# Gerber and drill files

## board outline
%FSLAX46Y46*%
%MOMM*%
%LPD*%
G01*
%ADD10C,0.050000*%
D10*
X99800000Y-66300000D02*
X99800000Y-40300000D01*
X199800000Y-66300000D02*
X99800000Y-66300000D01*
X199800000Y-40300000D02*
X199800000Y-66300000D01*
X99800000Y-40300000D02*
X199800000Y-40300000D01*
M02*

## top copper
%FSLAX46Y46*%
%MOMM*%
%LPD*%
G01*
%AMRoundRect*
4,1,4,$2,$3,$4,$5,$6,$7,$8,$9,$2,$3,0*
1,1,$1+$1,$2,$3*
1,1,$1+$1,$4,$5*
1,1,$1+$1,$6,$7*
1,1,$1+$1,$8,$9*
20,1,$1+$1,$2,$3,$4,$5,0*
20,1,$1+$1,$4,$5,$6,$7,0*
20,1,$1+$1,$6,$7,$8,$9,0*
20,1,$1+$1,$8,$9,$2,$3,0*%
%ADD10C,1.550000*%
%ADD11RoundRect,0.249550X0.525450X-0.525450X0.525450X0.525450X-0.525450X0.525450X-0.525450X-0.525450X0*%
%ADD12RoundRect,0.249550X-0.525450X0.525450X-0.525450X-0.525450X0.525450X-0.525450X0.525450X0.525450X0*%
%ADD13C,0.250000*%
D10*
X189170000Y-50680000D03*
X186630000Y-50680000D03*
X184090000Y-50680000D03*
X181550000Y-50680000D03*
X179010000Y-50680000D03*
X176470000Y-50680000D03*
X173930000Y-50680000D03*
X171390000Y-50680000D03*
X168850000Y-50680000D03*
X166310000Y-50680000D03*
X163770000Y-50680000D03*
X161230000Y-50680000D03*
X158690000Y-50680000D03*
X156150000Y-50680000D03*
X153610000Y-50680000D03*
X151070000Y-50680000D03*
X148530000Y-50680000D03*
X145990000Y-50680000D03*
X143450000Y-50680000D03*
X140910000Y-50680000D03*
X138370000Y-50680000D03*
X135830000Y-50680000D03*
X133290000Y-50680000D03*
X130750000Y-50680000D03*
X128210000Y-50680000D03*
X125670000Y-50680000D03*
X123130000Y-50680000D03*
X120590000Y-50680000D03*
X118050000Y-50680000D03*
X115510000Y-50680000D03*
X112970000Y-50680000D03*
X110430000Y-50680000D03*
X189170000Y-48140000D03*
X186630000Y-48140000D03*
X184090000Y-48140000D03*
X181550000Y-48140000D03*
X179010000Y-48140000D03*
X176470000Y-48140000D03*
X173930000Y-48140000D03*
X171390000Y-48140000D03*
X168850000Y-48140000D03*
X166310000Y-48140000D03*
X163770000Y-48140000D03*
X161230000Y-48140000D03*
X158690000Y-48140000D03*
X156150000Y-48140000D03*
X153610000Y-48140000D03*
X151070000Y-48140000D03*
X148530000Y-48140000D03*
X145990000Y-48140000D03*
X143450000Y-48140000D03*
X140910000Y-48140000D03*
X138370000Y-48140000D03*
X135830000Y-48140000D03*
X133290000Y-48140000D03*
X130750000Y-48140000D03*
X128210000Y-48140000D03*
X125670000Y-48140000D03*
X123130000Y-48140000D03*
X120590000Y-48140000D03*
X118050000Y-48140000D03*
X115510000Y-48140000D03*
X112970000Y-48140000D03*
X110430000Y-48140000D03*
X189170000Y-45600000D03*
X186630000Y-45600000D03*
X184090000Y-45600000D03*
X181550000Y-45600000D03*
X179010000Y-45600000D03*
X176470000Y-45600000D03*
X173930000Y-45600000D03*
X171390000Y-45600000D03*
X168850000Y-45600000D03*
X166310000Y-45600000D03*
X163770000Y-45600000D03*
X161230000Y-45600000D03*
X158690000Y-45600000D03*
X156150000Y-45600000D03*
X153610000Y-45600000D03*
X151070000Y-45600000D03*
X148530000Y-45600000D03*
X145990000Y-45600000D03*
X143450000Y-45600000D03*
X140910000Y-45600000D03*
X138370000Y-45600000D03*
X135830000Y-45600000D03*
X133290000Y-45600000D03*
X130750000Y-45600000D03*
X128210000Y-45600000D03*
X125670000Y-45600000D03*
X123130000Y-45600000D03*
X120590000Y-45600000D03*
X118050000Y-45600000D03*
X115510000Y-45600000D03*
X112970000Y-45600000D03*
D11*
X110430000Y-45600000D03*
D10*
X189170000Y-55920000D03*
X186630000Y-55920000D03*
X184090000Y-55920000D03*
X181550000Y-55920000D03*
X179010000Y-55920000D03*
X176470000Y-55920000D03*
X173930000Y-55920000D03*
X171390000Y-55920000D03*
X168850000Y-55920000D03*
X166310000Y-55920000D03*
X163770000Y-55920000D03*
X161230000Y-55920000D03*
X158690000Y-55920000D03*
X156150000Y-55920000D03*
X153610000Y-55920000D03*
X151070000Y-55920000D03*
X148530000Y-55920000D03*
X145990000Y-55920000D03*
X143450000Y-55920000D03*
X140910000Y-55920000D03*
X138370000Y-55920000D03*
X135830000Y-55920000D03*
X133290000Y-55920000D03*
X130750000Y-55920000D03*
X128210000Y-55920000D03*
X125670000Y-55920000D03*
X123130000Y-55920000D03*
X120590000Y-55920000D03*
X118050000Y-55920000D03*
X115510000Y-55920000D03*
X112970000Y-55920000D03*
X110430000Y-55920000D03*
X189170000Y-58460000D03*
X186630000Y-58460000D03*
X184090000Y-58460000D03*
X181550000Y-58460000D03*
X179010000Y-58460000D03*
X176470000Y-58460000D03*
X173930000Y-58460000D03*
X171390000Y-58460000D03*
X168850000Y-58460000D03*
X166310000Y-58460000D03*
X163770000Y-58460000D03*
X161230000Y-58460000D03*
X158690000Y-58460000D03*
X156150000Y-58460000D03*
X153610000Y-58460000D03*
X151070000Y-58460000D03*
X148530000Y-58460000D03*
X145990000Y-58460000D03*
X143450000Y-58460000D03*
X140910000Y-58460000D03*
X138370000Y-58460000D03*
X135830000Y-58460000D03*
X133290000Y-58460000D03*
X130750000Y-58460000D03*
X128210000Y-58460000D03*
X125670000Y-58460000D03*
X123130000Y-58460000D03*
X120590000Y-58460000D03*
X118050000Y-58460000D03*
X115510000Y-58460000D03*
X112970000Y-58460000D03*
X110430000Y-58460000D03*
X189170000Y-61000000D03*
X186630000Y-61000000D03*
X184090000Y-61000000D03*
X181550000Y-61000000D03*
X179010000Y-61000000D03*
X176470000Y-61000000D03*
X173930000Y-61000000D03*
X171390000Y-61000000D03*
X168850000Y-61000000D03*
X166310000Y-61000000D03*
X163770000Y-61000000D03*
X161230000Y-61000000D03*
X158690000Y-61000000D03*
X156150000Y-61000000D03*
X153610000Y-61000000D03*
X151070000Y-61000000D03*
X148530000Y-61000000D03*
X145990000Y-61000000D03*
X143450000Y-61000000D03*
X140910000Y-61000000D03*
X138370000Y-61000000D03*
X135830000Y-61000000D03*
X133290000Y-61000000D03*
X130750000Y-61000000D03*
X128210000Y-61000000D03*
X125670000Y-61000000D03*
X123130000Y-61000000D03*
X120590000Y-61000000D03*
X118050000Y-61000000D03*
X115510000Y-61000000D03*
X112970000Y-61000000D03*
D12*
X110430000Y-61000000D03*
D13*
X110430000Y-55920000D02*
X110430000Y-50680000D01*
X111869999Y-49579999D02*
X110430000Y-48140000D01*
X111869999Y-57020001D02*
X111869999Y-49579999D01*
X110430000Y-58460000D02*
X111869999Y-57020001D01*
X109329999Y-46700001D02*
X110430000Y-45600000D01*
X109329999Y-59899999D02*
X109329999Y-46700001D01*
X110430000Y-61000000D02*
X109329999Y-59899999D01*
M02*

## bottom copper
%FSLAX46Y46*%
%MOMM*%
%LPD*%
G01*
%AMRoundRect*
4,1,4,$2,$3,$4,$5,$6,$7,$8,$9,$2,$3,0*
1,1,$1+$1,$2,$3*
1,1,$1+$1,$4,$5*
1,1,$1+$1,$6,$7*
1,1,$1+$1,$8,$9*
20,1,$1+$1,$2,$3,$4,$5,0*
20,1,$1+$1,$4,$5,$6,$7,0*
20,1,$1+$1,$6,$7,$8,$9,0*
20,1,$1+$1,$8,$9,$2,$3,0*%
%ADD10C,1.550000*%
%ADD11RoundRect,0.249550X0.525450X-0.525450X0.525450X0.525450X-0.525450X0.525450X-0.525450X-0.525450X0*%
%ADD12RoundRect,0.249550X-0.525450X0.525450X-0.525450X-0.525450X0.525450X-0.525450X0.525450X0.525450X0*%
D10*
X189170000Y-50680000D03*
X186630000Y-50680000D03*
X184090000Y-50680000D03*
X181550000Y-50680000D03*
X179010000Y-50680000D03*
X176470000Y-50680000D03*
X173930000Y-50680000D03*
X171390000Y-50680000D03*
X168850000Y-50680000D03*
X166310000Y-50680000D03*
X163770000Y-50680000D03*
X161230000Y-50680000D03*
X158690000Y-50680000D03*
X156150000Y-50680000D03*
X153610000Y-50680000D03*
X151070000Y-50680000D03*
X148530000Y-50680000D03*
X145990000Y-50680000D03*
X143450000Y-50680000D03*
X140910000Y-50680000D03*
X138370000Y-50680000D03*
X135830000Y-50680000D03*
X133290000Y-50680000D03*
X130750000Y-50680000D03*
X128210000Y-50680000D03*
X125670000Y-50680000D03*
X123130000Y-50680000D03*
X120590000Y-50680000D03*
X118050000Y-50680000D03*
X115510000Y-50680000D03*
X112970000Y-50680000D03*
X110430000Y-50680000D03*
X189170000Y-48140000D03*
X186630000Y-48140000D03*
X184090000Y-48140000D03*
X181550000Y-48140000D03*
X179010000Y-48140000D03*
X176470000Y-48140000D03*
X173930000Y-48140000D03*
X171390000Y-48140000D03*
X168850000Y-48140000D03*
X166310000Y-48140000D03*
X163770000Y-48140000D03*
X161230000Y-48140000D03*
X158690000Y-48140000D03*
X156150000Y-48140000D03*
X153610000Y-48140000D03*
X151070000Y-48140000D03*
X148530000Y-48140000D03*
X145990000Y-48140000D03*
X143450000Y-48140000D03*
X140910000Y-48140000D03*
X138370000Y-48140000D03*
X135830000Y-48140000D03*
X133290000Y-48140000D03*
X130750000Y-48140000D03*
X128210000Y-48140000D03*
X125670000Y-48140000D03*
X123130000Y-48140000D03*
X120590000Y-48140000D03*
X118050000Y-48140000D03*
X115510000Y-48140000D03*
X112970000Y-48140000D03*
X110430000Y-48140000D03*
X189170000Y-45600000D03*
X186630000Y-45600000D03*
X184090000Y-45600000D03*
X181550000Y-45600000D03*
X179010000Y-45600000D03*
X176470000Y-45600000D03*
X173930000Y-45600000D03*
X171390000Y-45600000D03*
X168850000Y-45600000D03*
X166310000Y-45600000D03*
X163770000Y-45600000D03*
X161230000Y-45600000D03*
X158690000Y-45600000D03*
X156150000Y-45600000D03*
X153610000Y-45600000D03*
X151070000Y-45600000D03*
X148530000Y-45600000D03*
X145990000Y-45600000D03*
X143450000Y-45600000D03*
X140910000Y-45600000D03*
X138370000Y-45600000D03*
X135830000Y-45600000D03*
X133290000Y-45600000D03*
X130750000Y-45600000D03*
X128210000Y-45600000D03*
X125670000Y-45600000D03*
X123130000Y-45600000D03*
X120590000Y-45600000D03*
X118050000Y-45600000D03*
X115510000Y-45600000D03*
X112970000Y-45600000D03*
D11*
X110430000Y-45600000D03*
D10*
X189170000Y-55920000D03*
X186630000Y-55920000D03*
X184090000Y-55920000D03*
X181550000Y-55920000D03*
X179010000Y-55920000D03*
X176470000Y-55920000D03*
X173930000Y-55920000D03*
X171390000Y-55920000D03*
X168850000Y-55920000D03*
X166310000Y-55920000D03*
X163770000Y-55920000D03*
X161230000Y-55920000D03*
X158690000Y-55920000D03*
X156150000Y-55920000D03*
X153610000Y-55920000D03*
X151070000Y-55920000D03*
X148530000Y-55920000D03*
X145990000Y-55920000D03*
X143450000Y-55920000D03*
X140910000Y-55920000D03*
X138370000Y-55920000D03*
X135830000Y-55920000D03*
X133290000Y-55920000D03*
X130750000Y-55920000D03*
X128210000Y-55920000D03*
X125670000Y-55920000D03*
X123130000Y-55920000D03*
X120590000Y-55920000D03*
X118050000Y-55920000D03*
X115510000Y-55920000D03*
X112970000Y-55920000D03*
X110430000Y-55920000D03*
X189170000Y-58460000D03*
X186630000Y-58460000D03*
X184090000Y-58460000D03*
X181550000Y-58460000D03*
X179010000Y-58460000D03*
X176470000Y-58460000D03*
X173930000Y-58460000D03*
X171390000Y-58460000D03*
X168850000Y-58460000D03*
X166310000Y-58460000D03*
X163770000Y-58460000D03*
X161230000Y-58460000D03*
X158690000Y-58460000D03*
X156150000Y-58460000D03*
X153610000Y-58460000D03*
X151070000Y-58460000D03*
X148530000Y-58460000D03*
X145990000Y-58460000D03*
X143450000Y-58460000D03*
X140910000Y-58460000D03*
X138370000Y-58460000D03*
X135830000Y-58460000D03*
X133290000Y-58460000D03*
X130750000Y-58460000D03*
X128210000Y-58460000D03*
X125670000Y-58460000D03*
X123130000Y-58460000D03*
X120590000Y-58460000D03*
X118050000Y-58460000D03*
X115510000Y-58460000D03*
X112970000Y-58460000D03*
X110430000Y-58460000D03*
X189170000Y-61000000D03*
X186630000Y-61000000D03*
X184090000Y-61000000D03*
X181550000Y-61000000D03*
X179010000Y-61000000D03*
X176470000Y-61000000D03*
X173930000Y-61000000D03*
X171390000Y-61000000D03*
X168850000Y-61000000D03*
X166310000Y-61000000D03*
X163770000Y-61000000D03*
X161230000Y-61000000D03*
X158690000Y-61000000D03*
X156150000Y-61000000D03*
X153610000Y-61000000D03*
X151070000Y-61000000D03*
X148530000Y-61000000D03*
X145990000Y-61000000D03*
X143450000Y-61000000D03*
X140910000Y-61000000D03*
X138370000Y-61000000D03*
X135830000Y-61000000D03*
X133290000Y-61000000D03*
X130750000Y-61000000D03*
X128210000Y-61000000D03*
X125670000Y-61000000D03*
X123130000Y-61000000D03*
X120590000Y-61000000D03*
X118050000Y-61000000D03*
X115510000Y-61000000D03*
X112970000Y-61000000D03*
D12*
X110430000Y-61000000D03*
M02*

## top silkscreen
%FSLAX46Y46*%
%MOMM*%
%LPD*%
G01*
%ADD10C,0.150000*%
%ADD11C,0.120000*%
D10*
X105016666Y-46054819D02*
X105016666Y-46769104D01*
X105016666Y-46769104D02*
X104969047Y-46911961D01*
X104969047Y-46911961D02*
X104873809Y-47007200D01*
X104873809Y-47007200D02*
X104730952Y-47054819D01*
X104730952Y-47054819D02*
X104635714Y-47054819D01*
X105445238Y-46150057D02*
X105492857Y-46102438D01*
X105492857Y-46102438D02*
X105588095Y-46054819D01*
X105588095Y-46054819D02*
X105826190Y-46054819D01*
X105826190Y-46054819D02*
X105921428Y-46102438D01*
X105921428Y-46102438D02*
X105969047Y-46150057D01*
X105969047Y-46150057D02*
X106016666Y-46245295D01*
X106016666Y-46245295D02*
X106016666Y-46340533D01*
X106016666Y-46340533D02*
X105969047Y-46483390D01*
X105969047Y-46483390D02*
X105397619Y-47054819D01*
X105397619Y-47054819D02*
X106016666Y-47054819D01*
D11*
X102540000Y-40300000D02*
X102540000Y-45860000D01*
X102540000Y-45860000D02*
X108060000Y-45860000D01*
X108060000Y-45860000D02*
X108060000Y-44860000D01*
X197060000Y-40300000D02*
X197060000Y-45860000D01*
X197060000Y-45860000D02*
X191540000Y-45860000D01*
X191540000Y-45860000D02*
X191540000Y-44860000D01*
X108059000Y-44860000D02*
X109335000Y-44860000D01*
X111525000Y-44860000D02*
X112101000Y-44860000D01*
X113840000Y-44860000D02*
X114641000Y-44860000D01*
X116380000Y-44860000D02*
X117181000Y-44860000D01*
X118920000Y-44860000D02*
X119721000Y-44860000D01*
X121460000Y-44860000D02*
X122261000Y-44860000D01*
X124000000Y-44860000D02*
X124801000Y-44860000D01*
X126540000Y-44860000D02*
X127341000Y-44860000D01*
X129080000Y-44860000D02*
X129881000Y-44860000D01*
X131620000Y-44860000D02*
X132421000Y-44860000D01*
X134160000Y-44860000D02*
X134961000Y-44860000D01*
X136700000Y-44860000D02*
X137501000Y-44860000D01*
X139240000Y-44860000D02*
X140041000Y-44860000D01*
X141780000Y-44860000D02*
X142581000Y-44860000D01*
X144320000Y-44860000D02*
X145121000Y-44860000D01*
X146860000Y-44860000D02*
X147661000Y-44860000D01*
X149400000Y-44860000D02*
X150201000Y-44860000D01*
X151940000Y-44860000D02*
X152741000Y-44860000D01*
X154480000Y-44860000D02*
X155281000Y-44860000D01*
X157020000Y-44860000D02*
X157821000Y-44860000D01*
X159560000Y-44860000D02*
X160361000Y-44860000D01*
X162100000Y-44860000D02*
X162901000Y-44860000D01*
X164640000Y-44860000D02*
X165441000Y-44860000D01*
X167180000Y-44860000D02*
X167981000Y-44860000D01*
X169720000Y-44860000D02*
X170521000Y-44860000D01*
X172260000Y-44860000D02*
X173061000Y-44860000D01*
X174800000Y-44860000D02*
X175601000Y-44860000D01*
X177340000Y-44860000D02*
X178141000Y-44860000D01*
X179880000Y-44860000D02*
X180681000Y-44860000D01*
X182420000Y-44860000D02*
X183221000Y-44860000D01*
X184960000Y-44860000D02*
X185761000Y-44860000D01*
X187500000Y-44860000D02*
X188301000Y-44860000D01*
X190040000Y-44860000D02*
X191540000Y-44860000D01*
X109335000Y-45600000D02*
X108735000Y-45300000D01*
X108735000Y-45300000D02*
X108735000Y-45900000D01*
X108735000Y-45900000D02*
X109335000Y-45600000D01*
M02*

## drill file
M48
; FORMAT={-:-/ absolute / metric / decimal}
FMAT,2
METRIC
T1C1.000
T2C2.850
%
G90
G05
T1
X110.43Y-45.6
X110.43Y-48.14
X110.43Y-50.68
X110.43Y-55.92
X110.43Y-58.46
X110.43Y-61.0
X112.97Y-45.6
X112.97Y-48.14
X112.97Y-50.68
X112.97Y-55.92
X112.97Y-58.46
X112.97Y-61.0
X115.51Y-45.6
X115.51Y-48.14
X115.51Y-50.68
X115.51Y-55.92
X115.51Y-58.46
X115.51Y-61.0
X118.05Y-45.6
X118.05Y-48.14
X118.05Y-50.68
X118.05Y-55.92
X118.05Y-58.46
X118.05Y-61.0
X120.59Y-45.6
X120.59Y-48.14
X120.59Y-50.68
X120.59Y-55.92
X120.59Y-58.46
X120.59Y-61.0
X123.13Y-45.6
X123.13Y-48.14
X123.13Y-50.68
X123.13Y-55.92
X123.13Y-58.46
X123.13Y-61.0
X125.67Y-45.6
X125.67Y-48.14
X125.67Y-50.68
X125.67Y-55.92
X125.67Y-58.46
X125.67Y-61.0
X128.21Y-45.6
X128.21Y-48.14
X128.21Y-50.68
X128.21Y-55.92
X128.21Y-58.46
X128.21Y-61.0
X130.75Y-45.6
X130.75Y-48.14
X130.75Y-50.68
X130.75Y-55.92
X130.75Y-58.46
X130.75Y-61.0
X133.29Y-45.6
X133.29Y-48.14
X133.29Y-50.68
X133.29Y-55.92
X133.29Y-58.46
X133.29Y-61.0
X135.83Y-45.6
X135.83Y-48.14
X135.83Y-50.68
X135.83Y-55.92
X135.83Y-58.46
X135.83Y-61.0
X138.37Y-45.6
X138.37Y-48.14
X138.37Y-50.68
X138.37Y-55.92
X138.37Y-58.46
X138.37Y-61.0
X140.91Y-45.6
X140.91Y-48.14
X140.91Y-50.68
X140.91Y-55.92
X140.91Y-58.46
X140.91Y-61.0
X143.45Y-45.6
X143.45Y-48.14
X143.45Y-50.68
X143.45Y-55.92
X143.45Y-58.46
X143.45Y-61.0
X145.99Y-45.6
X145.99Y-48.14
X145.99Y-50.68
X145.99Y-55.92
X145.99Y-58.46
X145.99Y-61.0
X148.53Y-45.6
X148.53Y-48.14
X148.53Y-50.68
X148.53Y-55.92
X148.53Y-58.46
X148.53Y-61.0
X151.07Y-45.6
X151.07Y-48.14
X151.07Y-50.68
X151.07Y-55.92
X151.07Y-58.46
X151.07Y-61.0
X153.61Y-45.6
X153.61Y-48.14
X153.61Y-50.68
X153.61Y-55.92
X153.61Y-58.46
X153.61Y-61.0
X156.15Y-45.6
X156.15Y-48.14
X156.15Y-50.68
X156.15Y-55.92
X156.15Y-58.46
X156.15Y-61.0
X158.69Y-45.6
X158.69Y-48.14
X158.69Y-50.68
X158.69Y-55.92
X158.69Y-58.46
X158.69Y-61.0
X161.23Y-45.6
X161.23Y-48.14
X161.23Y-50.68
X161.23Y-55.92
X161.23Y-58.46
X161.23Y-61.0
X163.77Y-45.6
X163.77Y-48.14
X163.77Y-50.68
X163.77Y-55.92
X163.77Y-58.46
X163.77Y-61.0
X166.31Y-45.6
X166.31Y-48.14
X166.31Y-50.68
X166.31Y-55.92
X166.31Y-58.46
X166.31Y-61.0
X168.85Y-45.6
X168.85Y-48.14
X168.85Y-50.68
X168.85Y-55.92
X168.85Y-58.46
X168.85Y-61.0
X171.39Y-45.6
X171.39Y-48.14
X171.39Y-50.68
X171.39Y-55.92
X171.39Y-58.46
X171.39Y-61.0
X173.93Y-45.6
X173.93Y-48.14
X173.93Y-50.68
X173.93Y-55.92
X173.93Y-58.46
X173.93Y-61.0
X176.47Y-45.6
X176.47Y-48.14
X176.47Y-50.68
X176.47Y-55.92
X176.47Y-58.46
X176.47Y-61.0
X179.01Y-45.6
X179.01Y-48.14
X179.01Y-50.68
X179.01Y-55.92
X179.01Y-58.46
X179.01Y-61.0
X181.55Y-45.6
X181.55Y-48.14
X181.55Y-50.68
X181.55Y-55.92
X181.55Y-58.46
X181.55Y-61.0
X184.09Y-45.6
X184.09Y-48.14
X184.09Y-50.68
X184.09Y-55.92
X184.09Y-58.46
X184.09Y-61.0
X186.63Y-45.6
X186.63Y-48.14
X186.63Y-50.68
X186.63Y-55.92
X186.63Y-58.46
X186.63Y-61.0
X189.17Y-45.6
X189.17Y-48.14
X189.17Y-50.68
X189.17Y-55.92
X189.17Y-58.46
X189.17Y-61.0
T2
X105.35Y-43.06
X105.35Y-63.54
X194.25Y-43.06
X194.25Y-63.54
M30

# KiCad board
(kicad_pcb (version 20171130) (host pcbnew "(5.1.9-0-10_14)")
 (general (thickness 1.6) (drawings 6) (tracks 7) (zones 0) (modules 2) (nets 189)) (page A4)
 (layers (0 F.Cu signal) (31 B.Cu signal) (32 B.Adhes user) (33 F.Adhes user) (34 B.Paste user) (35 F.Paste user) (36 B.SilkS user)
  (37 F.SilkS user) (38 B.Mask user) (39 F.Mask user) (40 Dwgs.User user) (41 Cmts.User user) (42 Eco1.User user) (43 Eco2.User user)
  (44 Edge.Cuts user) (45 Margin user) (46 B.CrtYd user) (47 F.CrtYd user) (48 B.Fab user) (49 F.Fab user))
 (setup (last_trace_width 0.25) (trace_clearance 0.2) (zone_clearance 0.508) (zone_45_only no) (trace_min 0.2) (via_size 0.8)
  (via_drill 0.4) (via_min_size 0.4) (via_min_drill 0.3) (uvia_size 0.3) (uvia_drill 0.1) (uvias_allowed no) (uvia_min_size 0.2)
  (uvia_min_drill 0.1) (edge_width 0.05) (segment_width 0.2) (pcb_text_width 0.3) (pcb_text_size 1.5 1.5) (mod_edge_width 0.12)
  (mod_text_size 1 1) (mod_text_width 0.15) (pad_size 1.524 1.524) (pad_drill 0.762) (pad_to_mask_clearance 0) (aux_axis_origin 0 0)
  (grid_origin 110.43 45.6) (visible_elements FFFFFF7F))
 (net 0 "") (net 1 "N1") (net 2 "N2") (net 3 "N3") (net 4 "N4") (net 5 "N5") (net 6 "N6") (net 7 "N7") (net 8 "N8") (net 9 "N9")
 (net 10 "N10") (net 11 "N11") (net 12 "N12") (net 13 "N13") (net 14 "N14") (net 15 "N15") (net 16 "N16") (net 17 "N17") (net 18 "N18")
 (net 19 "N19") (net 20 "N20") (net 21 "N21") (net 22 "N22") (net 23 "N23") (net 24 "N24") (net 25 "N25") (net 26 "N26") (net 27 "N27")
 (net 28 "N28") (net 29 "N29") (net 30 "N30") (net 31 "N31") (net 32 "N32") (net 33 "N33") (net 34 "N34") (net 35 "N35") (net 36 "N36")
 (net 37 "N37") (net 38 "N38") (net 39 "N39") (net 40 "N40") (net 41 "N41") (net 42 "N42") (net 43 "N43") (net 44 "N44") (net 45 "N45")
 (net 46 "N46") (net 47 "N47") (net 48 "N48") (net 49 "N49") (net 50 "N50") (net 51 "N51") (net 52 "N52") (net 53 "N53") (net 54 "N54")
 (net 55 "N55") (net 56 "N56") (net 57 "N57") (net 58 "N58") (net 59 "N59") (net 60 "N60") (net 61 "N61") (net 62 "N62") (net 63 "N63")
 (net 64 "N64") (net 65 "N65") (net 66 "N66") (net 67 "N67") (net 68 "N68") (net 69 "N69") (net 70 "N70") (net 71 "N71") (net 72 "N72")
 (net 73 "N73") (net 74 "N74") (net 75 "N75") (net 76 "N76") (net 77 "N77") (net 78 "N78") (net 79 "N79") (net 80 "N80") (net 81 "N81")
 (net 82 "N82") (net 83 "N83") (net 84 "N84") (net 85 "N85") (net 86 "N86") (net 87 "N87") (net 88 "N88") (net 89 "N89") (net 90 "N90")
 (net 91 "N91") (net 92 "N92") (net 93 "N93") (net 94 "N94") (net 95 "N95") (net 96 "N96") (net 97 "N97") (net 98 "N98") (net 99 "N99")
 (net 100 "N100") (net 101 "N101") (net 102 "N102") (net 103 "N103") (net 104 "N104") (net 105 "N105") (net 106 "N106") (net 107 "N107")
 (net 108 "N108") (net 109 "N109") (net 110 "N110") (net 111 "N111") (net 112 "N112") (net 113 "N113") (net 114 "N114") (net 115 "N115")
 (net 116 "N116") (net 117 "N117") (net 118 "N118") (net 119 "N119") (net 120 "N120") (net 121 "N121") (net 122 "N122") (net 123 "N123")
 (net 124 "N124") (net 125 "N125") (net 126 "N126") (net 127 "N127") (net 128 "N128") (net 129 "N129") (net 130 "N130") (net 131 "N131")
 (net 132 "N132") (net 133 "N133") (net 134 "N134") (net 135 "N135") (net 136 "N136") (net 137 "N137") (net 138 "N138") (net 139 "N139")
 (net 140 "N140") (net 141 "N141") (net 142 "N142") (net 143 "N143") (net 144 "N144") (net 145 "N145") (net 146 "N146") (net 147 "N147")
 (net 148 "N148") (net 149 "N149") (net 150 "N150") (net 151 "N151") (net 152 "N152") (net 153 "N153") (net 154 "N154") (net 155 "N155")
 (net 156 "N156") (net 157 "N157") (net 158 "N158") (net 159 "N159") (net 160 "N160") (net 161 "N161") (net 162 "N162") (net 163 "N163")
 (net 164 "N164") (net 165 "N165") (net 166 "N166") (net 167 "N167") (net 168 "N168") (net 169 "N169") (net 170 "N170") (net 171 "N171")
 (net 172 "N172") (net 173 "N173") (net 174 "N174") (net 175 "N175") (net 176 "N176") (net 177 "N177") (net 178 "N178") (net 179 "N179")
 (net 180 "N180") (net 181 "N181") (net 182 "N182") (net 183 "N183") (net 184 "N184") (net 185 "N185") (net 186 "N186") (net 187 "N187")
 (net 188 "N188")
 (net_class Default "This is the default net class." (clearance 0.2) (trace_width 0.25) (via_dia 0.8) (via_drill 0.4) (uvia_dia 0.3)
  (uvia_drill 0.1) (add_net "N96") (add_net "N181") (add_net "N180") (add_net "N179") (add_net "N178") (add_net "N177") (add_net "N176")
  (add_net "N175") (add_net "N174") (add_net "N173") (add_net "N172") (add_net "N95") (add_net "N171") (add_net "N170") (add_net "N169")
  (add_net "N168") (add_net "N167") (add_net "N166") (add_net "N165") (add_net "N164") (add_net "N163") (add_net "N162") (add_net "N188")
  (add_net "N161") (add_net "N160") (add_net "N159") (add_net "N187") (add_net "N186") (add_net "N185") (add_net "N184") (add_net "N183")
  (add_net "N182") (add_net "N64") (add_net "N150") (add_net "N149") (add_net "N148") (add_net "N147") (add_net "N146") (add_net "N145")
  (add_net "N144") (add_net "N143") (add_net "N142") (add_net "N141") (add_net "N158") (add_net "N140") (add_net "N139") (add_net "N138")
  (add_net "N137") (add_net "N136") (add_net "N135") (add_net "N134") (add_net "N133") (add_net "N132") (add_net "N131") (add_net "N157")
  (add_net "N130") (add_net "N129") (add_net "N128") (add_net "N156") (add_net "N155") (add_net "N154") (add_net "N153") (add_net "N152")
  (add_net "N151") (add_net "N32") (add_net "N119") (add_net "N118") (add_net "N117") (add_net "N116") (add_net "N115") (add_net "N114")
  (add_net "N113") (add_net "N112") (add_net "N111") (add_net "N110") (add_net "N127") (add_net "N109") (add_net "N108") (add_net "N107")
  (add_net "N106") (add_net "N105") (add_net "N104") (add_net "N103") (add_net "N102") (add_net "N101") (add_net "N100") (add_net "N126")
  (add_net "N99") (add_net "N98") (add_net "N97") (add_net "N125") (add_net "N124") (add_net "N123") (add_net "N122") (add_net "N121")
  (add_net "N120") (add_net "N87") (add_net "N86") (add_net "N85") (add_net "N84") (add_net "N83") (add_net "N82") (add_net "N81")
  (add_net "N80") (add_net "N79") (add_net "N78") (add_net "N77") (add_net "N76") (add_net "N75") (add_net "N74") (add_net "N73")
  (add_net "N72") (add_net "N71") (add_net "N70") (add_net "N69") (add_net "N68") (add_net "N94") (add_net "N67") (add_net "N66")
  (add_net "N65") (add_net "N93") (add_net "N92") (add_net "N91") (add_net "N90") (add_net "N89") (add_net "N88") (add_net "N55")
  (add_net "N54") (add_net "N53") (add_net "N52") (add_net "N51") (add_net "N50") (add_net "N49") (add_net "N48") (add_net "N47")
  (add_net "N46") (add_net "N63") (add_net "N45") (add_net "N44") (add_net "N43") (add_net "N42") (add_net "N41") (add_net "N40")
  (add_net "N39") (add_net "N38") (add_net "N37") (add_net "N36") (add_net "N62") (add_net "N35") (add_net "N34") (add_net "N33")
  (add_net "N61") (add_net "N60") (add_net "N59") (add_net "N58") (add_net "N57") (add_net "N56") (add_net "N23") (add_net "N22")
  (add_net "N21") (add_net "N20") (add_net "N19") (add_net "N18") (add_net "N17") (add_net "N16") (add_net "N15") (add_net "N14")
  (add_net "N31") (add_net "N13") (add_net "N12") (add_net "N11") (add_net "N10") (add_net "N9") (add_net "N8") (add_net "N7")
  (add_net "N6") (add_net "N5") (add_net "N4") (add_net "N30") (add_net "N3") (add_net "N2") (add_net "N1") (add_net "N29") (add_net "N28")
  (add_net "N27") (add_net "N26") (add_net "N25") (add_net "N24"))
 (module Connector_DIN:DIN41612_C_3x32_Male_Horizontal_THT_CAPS (layer F.Cu) (at 110.43 45.6)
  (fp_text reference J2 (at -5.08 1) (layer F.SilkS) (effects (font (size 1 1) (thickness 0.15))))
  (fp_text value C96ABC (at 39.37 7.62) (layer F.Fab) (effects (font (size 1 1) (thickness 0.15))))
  (fp_line (start -7.89 -5.3) (end -7.89 0.26) (layer F.SilkS) (width 0.12))
  (fp_line (start -7.89 0.26) (end -2.37 0.26) (layer F.SilkS) (width 0.12))
  (fp_line (start -2.37 0.26) (end -2.37 -0.74) (layer F.SilkS) (width 0.12))
  (fp_line (start 86.63 -5.3) (end 86.63 0.26) (layer F.SilkS) (width 0.12))
  (fp_line (start 86.63 0.26) (end 81.11 0.26) (layer F.SilkS) (width 0.12))
  (fp_line (start 81.11 0.26) (end 81.11 -0.74) (layer F.SilkS) (width 0.12))
  (fp_line (start -2.371 -0.74) (end -1.095 -0.74) (layer F.SilkS) (width 0.12))
  (fp_line (start 1.095 -0.74) (end 1.671 -0.74) (layer F.SilkS) (width 0.12))
  (fp_line (start 3.41 -0.74) (end 4.211 -0.74) (layer F.SilkS) (width 0.12))
  (fp_line (start 5.95 -0.74) (end 6.751 -0.74) (layer F.SilkS) (width 0.12))
  (fp_line (start 8.49 -0.74) (end 9.291 -0.74) (layer F.SilkS) (width 0.12))
  (fp_line (start 11.03 -0.74) (end 11.831 -0.74) (layer F.SilkS) (width 0.12))
  (fp_line (start 13.57 -0.74) (end 14.371 -0.74) (layer F.SilkS) (width 0.12))
  (fp_line (start 16.11 -0.74) (end 16.911 -0.74) (layer F.SilkS) (width 0.12))
  (fp_line (start 18.65 -0.74) (end 19.451 -0.74) (layer F.SilkS) (width 0.12))
  (fp_line (start 21.19 -0.74) (end 21.991 -0.74) (layer F.SilkS) (width 0.12))
  (fp_line (start 23.73 -0.74) (end 24.531 -0.74) (layer F.SilkS) (width 0.12))
  (fp_line (start 26.27 -0.74) (end 27.071 -0.74) (layer F.SilkS) (width 0.12))
  (fp_line (start 28.81 -0.74) (end 29.611 -0.74) (layer F.SilkS) (width 0.12))
  (fp_line (start 31.35 -0.74) (end 32.151 -0.74) (layer F.SilkS) (width 0.12))
  (fp_line (start 33.89 -0.74) (end 34.691 -0.74) (layer F.SilkS) (width 0.12))
  (fp_line (start 36.43 -0.74) (end 37.231 -0.74) (layer F.SilkS) (width 0.12))
  (fp_line (start 38.97 -0.74) (end 39.771 -0.74) (layer F.SilkS) (width 0.12))
  (fp_line (start 41.51 -0.74) (end 42.311 -0.74) (layer F.SilkS) (width 0.12))
  (fp_line (start 44.05 -0.74) (end 44.851 -0.74) (layer F.SilkS) (width 0.12))
  (fp_line (start 46.59 -0.74) (end 47.391 -0.74) (layer F.SilkS) (width 0.12))
  (fp_line (start 49.13 -0.74) (end 49.931 -0.74) (layer F.SilkS) (width 0.12))
  (fp_line (start 51.67 -0.74) (end 52.471 -0.74) (layer F.SilkS) (width 0.12))
  (fp_line (start 54.21 -0.74) (end 55.011 -0.74) (layer F.SilkS) (width 0.12))
  (fp_line (start 56.75 -0.74) (end 57.551 -0.74) (layer F.SilkS) (width 0.12))
  (fp_line (start 59.29 -0.74) (end 60.091 -0.74) (layer F.SilkS) (width 0.12))
  (fp_line (start 61.83 -0.74) (end 62.631 -0.74) (layer F.SilkS) (width 0.12))
  (fp_line (start 64.37 -0.74) (end 65.171 -0.74) (layer F.SilkS) (width 0.12))
  (fp_line (start 66.91 -0.74) (end 67.711 -0.74) (layer F.SilkS) (width 0.12))
  (fp_line (start 69.45 -0.74) (end 70.251 -0.74) (layer F.SilkS) (width 0.12))
  (fp_line (start 71.99 -0.74) (end 72.791 -0.74) (layer F.SilkS) (width 0.12))
  (fp_line (start 74.53 -0.74) (end 75.331 -0.74) (layer F.SilkS) (width 0.12))
  (fp_line (start 77.07 -0.74) (end 77.871 -0.74) (layer F.SilkS) (width 0.12))
  (fp_line (start 79.61 -0.74) (end 81.11 -0.74) (layer F.SilkS) (width 0.12))
  (fp_line (start -1.095 0) (end -1.695 -0.3) (layer F.SilkS) (width 0.12))
  (fp_line (start -1.695 -0.3) (end -1.695 0.3) (layer F.SilkS) (width 0.12))
  (fp_line (start -1.695 0.3) (end -1.095 0) (layer F.SilkS) (width 0.12))
  (pad C32 thru_hole circle (at 78.74 5.08) (size 1.55 1.55) (drill 1) (layers *.Cu *.Mask) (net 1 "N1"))
  (pad C31 thru_hole circle (at 76.2 5.08) (size 1.55 1.55) (drill 1) (layers *.Cu *.Mask) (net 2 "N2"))
  (pad C30 thru_hole circle (at 73.66 5.08) (size 1.55 1.55) (drill 1) (layers *.Cu *.Mask) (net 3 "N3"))
  (pad C29 thru_hole circle (at 71.12 5.08) (size 1.55 1.55) (drill 1) (layers *.Cu *.Mask) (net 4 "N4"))
  (pad C28 thru_hole circle (at 68.58 5.08) (size 1.55 1.55) (drill 1) (layers *.Cu *.Mask) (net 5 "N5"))
  (pad C27 thru_hole circle (at 66.04 5.08) (size 1.55 1.55) (drill 1) (layers *.Cu *.Mask) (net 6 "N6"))
  (pad C26 thru_hole circle (at 63.5 5.08) (size 1.55 1.55) (drill 1) (layers *.Cu *.Mask) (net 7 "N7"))
  (pad C25 thru_hole circle (at 60.96 5.08) (size 1.55 1.55) (drill 1) (layers *.Cu *.Mask) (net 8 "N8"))
  (pad C24 thru_hole circle (at 58.42 5.08) (size 1.55 1.55) (drill 1) (layers *.Cu *.Mask) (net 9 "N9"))
  (pad C23 thru_hole circle (at 55.88 5.08) (size 1.55 1.55) (drill 1) (layers *.Cu *.Mask) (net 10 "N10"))
  (pad C22 thru_hole circle (at 53.34 5.08) (size 1.55 1.55) (drill 1) (layers *.Cu *.Mask) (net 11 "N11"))
  (pad C21 thru_hole circle (at 50.8 5.08) (size 1.55 1.55) (drill 1) (layers *.Cu *.Mask) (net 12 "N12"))
  (pad C20 thru_hole circle (at 48.26 5.08) (size 1.55 1.55) (drill 1) (layers *.Cu *.Mask) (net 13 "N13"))
  (pad C19 thru_hole circle (at 45.72 5.08) (size 1.55 1.55) (drill 1) (layers *.Cu *.Mask) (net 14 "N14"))
  (pad C18 thru_hole circle (at 43.18 5.08) (size 1.55 1.55) (drill 1) (layers *.Cu *.Mask) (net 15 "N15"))
  (pad C17 thru_hole circle (at 40.64 5.08) (size 1.55 1.55) (drill 1) (layers *.Cu *.Mask) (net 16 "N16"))
  (pad C16 thru_hole circle (at 38.1 5.08) (size 1.55 1.55) (drill 1) (layers *.Cu *.Mask) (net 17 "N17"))
  (pad C15 thru_hole circle (at 35.56 5.08) (size 1.55 1.55) (drill 1) (layers *.Cu *.Mask) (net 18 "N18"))
  (pad C14 thru_hole circle (at 33.02 5.08) (size 1.55 1.55) (drill 1) (layers *.Cu *.Mask) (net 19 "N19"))
  (pad C13 thru_hole circle (at 30.48 5.08) (size 1.55 1.55) (drill 1) (layers *.Cu *.Mask) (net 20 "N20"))
  (pad C12 thru_hole circle (at 27.94 5.08) (size 1.55 1.55) (drill 1) (layers *.Cu *.Mask) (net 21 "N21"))
  (pad C11 thru_hole circle (at 25.4 5.08) (size 1.55 1.55) (drill 1) (layers *.Cu *.Mask) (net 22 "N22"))
  (pad C10 thru_hole circle (at 22.86 5.08) (size 1.55 1.55) (drill 1) (layers *.Cu *.Mask) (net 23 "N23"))
  (pad C9 thru_hole circle (at 20.32 5.08) (size 1.55 1.55) (drill 1) (layers *.Cu *.Mask) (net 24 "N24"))
  (pad C8 thru_hole circle (at 17.78 5.08) (size 1.55 1.55) (drill 1) (layers *.Cu *.Mask) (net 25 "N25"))
  (pad C7 thru_hole circle (at 15.24 5.08) (size 1.55 1.55) (drill 1) (layers *.Cu *.Mask) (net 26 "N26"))
  (pad C6 thru_hole circle (at 12.7 5.08) (size 1.55 1.55) (drill 1) (layers *.Cu *.Mask) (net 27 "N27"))
  (pad C5 thru_hole circle (at 10.16 5.08) (size 1.55 1.55) (drill 1) (layers *.Cu *.Mask) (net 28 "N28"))
  (pad C4 thru_hole circle (at 7.62 5.08) (size 1.55 1.55) (drill 1) (layers *.Cu *.Mask) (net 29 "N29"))
  (pad C3 thru_hole circle (at 5.08 5.08) (size 1.55 1.55) (drill 1) (layers *.Cu *.Mask) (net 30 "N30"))
  (pad C2 thru_hole circle (at 2.54 5.08) (size 1.55 1.55) (drill 1) (layers *.Cu *.Mask) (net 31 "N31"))
  (pad C1 thru_hole circle (at 0 5.08) (size 1.55 1.55) (drill 1) (layers *.Cu *.Mask) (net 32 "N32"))
  (pad B32 thru_hole circle (at 78.74 2.54) (size 1.55 1.55) (drill 1) (layers *.Cu *.Mask) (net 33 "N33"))
  (pad B31 thru_hole circle (at 76.2 2.54) (size 1.55 1.55) (drill 1) (layers *.Cu *.Mask) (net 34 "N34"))
  (pad B30 thru_hole circle (at 73.66 2.54) (size 1.55 1.55) (drill 1) (layers *.Cu *.Mask) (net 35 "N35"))
  (pad B29 thru_hole circle (at 71.12 2.54) (size 1.55 1.55) (drill 1) (layers *.Cu *.Mask) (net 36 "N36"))
  (pad B28 thru_hole circle (at 68.58 2.54) (size 1.55 1.55) (drill 1) (layers *.Cu *.Mask) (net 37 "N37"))
  (pad B27 thru_hole circle (at 66.04 2.54) (size 1.55 1.55) (drill 1) (layers *.Cu *.Mask) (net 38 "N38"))
  (pad B26 thru_hole circle (at 63.5 2.54) (size 1.55 1.55) (drill 1) (layers *.Cu *.Mask) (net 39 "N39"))
  (pad B25 thru_hole circle (at 60.96 2.54) (size 1.55 1.55) (drill 1) (layers *.Cu *.Mask) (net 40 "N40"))
  (pad B24 thru_hole circle (at 58.42 2.54) (size 1.55 1.55) (drill 1) (layers *.Cu *.Mask) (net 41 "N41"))
  (pad B23 thru_hole circle (at 55.88 2.54) (size 1.55 1.55) (drill 1) (layers *.Cu *.Mask) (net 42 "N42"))
  (pad B22 thru_hole circle (at 53.34 2.54) (size 1.55 1.55) (drill 1) (layers *.Cu *.Mask) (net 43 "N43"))
  (pad B21 thru_hole circle (at 50.8 2.54) (size 1.55 1.55) (drill 1) (layers *.Cu *.Mask) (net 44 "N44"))
  (pad B20 thru_hole circle (at 48.26 2.54) (size 1.55 1.55) (drill 1) (layers *.Cu *.Mask) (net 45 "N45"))
  (pad B19 thru_hole circle (at 45.72 2.54) (size 1.55 1.55) (drill 1) (layers *.Cu *.Mask) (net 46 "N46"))
  (pad B18 thru_hole circle (at 43.18 2.54) (size 1.55 1.55) (drill 1) (layers *.Cu *.Mask) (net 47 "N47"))
  (pad B17 thru_hole circle (at 40.64 2.54) (size 1.55 1.55) (drill 1) (layers *.Cu *.Mask) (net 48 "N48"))
  (pad B16 thru_hole circle (at 38.1 2.54) (size 1.55 1.55) (drill 1) (layers *.Cu *.Mask) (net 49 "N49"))
  (pad B15 thru_hole circle (at 35.56 2.54) (size 1.55 1.55) (drill 1) (layers *.Cu *.Mask) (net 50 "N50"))
  (pad B14 thru_hole circle (at 33.02 2.54) (size 1.55 1.55) (drill 1) (layers *.Cu *.Mask) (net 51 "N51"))
  (pad B13 thru_hole circle (at 30.48 2.54) (size 1.55 1.55) (drill 1) (layers *.Cu *.Mask) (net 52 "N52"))
  (pad B12 thru_hole circle (at 27.94 2.54) (size 1.55 1.55) (drill 1) (layers *.Cu *.Mask) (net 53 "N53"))
  (pad B11 thru_hole circle (at 25.4 2.54) (size 1.55 1.55) (drill 1) (layers *.Cu *.Mask) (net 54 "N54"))
  (pad B10 thru_hole circle (at 22.86 2.54) (size 1.55 1.55) (drill 1) (layers *.Cu *.Mask) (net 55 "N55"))
  (pad B9 thru_hole circle (at 20.32 2.54) (size 1.55 1.55) (drill 1) (layers *.Cu *.Mask) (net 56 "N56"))
  (pad B8 thru_hole circle (at 17.78 2.54) (size 1.55 1.55) (drill 1) (layers *.Cu *.Mask) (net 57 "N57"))
  (pad B7 thru_hole circle (at 15.24 2.54) (size 1.55 1.55) (drill 1) (layers *.Cu *.Mask) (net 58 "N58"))
  (pad B6 thru_hole circle (at 12.7 2.54) (size 1.55 1.55) (drill 1) (layers *.Cu *.Mask) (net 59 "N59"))
  (pad B5 thru_hole circle (at 10.16 2.54) (size 1.55 1.55) (drill 1) (layers *.Cu *.Mask) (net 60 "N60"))
  (pad B4 thru_hole circle (at 7.62 2.54) (size 1.55 1.55) (drill 1) (layers *.Cu *.Mask) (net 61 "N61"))
  (pad B3 thru_hole circle (at 5.08 2.54) (size 1.55 1.55) (drill 1) (layers *.Cu *.Mask) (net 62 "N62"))
  (pad B2 thru_hole circle (at 2.54 2.54) (size 1.55 1.55) (drill 1) (layers *.Cu *.Mask) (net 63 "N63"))
  (pad B1 thru_hole circle (at 0 2.54) (size 1.55 1.55) (drill 1) (layers *.Cu *.Mask) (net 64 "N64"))
  (pad A32 thru_hole circle (at 78.74 0) (size 1.55 1.55) (drill 1) (layers *.Cu *.Mask) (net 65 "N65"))
  (pad A31 thru_hole circle (at 76.2 0) (size 1.55 1.55) (drill 1) (layers *.Cu *.Mask) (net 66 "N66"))
  (pad A30 thru_hole circle (at 73.66 0) (size 1.55 1.55) (drill 1) (layers *.Cu *.Mask) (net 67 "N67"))
  (pad A29 thru_hole circle (at 71.12 0) (size 1.55 1.55) (drill 1) (layers *.Cu *.Mask) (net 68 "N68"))
  (pad A28 thru_hole circle (at 68.58 0) (size 1.55 1.55) (drill 1) (layers *.Cu *.Mask) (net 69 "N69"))
  (pad A27 thru_hole circle (at 66.04 0) (size 1.55 1.55) (drill 1) (layers *.Cu *.Mask) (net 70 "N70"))
  (pad A26 thru_hole circle (at 63.5 0) (size 1.55 1.55) (drill 1) (layers *.Cu *.Mask) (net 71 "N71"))
  (pad A25 thru_hole circle (at 60.96 0) (size 1.55 1.55) (drill 1) (layers *.Cu *.Mask) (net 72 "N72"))
  (pad A24 thru_hole circle (at 58.42 0) (size 1.55 1.55) (drill 1) (layers *.Cu *.Mask) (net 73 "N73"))
  (pad A23 thru_hole circle (at 55.88 0) (size 1.55 1.55) (drill 1) (layers *.Cu *.Mask) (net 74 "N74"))
  (pad A22 thru_hole circle (at 53.34 0) (size 1.55 1.55) (drill 1) (layers *.Cu *.Mask) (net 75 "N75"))
  (pad A21 thru_hole circle (at 50.8 0) (size 1.55 1.55) (drill 1) (layers *.Cu *.Mask) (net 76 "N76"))
  (pad A20 thru_hole circle (at 48.26 0) (size 1.55 1.55) (drill 1) (layers *.Cu *.Mask) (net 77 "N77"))
  (pad A19 thru_hole circle (at 45.72 0) (size 1.55 1.55) (drill 1) (layers *.Cu *.Mask) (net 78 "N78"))
  (pad A18 thru_hole circle (at 43.18 0) (size 1.55 1.55) (drill 1) (layers *.Cu *.Mask) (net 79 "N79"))
  (pad A17 thru_hole circle (at 40.64 0) (size 1.55 1.55) (drill 1) (layers *.Cu *.Mask) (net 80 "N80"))
  (pad A16 thru_hole circle (at 38.1 0) (size 1.55 1.55) (drill 1) (layers *.Cu *.Mask) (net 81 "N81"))
  (pad A15 thru_hole circle (at 35.56 0) (size 1.55 1.55) (drill 1) (layers *.Cu *.Mask) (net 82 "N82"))
  (pad A14 thru_hole circle (at 33.02 0) (size 1.55 1.55) (drill 1) (layers *.Cu *.Mask) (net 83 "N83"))
  (pad A13 thru_hole circle (at 30.48 0) (size 1.55 1.55) (drill 1) (layers *.Cu *.Mask) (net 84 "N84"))
  (pad A12 thru_hole circle (at 27.94 0) (size 1.55 1.55) (drill 1) (layers *.Cu *.Mask) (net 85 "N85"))
  (pad A11 thru_hole circle (at 25.4 0) (size 1.55 1.55) (drill 1) (layers *.Cu *.Mask) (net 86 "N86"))
  (pad A10 thru_hole circle (at 22.86 0) (size 1.55 1.55) (drill 1) (layers *.Cu *.Mask) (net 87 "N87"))
  (pad A9 thru_hole circle (at 20.32 0) (size 1.55 1.55) (drill 1) (layers *.Cu *.Mask) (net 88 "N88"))
  (pad A8 thru_hole circle (at 17.78 0) (size 1.55 1.55) (drill 1) (layers *.Cu *.Mask) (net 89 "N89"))
  (pad A7 thru_hole circle (at 15.24 0) (size 1.55 1.55) (drill 1) (layers *.Cu *.Mask) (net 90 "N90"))
  (pad A6 thru_hole circle (at 12.7 0) (size 1.55 1.55) (drill 1) (layers *.Cu *.Mask) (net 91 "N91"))
  (pad A5 thru_hole circle (at 10.16 0) (size 1.55 1.55) (drill 1) (layers *.Cu *.Mask) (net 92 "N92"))
  (pad A4 thru_hole circle (at 7.62 0) (size 1.55 1.55) (drill 1) (layers *.Cu *.Mask) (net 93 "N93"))
  (pad A3 thru_hole circle (at 5.08 0) (size 1.55 1.55) (drill 1) (layers *.Cu *.Mask) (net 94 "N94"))
  (pad A2 thru_hole circle (at 2.54 0) (size 1.55 1.55) (drill 1) (layers *.Cu *.Mask) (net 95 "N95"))
  (pad A1 thru_hole roundrect (at 0 0 90) (size 1.55 1.55) (drill 1) (layers *.Cu *.Mask) (roundrect_rratio 0.161) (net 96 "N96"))
  (pad "" np_thru_hole circle (at 83.82 -2.54) (size 2.85 2.85) (drill 2.85) (layers *.Cu *.Mask))
  (pad "" np_thru_hole circle (at -5.08 -2.54) (size 2.85 2.85) (drill 2.85) (layers *.Cu *.Mask)))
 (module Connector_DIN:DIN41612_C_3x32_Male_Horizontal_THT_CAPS (layer B.Cu) (at 110.43 61)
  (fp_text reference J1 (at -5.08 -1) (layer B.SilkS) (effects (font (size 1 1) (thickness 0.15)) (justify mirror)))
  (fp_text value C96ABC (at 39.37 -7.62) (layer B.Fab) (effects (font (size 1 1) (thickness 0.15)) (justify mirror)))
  (pad C32 thru_hole circle (at 78.74 -5.08) (size 1.55 1.55) (drill 1) (layers *.Cu *.Mask) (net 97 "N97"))
  (pad C31 thru_hole circle (at 76.2 -5.08) (size 1.55 1.55) (drill 1) (layers *.Cu *.Mask) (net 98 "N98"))
  (pad C30 thru_hole circle (at 73.66 -5.08) (size 1.55 1.55) (drill 1) (layers *.Cu *.Mask) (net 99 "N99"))
  (pad C29 thru_hole circle (at 71.12 -5.08) (size 1.55 1.55) (drill 1) (layers *.Cu *.Mask) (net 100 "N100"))
  (pad C28 thru_hole circle (at 68.58 -5.08) (size 1.55 1.55) (drill 1) (layers *.Cu *.Mask) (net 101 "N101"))
  (pad C27 thru_hole circle (at 66.04 -5.08) (size 1.55 1.55) (drill 1) (layers *.Cu *.Mask) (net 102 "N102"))
  (pad C26 thru_hole circle (at 63.5 -5.08) (size 1.55 1.55) (drill 1) (layers *.Cu *.Mask) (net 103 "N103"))
  (pad C25 thru_hole circle (at 60.96 -5.08) (size 1.55 1.55) (drill 1) (layers *.Cu *.Mask) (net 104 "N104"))
  (pad C24 thru_hole circle (at 58.42 -5.08) (size 1.55 1.55) (drill 1) (layers *.Cu *.Mask) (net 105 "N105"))
  (pad C23 thru_hole circle (at 55.88 -5.08) (size 1.55 1.55) (drill 1) (layers *.Cu *.Mask) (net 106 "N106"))
  (pad C22 thru_hole circle (at 53.34 -5.08) (size 1.55 1.55) (drill 1) (layers *.Cu *.Mask) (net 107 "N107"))
  (pad C21 thru_hole circle (at 50.8 -5.08) (size 1.55 1.55) (drill 1) (layers *.Cu *.Mask) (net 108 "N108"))
  (pad C20 thru_hole circle (at 48.26 -5.08) (size 1.55 1.55) (drill 1) (layers *.Cu *.Mask) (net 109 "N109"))
  (pad C19 thru_hole circle (at 45.72 -5.08) (size 1.55 1.55) (drill 1) (layers *.Cu *.Mask) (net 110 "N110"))
  (pad C18 thru_hole circle (at 43.18 -5.08) (size 1.55 1.55) (drill 1) (layers *.Cu *.Mask) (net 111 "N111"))
  (pad C17 thru_hole circle (at 40.64 -5.08) (size 1.55 1.55) (drill 1) (layers *.Cu *.Mask) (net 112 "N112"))
  (pad C16 thru_hole circle (at 38.1 -5.08) (size 1.55 1.55) (drill 1) (layers *.Cu *.Mask) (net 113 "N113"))
  (pad C15 thru_hole circle (at 35.56 -5.08) (size 1.55 1.55) (drill 1) (layers *.Cu *.Mask) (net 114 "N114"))
  (pad C14 thru_hole circle (at 33.02 -5.08) (size 1.55 1.55) (drill 1) (layers *.Cu *.Mask) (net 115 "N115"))
  (pad C13 thru_hole circle (at 30.48 -5.08) (size 1.55 1.55) (drill 1) (layers *.Cu *.Mask) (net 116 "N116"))
  (pad C12 thru_hole circle (at 27.94 -5.08) (size 1.55 1.55) (drill 1) (layers *.Cu *.Mask) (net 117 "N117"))
  (pad C11 thru_hole circle (at 25.4 -5.08) (size 1.55 1.55) (drill 1) (layers *.Cu *.Mask) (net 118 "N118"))
  (pad C10 thru_hole circle (at 22.86 -5.08) (size 1.55 1.55) (drill 1) (layers *.Cu *.Mask) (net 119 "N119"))
  (pad C9 thru_hole circle (at 20.32 -5.08) (size 1.55 1.55) (drill 1) (layers *.Cu *.Mask) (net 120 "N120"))
  (pad C8 thru_hole circle (at 17.78 -5.08) (size 1.55 1.55) (drill 1) (layers *.Cu *.Mask) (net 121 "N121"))
  (pad C7 thru_hole circle (at 15.24 -5.08) (size 1.55 1.55) (drill 1) (layers *.Cu *.Mask) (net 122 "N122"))
  (pad C6 thru_hole circle (at 12.7 -5.08) (size 1.55 1.55) (drill 1) (layers *.Cu *.Mask) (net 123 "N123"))
  (pad C5 thru_hole circle (at 10.16 -5.08) (size 1.55 1.55) (drill 1) (layers *.Cu *.Mask) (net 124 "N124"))
  (pad C4 thru_hole circle (at 7.62 -5.08) (size 1.55 1.55) (drill 1) (layers *.Cu *.Mask) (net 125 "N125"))
  (pad C3 thru_hole circle (at 5.08 -5.08) (size 1.55 1.55) (drill 1) (layers *.Cu *.Mask) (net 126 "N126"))
  (pad C2 thru_hole circle (at 2.54 -5.08) (size 1.55 1.55) (drill 1) (layers *.Cu *.Mask) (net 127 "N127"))
  (pad C1 thru_hole circle (at 0 -5.08) (size 1.55 1.55) (drill 1) (layers *.Cu *.Mask) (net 32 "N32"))
  (pad B32 thru_hole circle (at 78.74 -2.54) (size 1.55 1.55) (drill 1) (layers *.Cu *.Mask) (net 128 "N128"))
  (pad B31 thru_hole circle (at 76.2 -2.54) (size 1.55 1.55) (drill 1) (layers *.Cu *.Mask) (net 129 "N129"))
  (pad B30 thru_hole circle (at 73.66 -2.54) (size 1.55 1.55) (drill 1) (layers *.Cu *.Mask) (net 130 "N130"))
  (pad B29 thru_hole circle (at 71.12 -2.54) (size 1.55 1.55) (drill 1) (layers *.Cu *.Mask) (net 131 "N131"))
  (pad B28 thru_hole circle (at 68.58 -2.54) (size 1.55 1.55) (drill 1) (layers *.Cu *.Mask) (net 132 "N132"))
  (pad B27 thru_hole circle (at 66.04 -2.54) (size 1.55 1.55) (drill 1) (layers *.Cu *.Mask) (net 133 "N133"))
  (pad B26 thru_hole circle (at 63.5 -2.54) (size 1.55 1.55) (drill 1) (layers *.Cu *.Mask) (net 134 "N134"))
  (pad B25 thru_hole circle (at 60.96 -2.54) (size 1.55 1.55) (drill 1) (layers *.Cu *.Mask) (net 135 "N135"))
  (pad B24 thru_hole circle (at 58.42 -2.54) (size 1.55 1.55) (drill 1) (layers *.Cu *.Mask) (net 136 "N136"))
  (pad B23 thru_hole circle (at 55.88 -2.54) (size 1.55 1.55) (drill 1) (layers *.Cu *.Mask) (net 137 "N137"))
  (pad B22 thru_hole circle (at 53.34 -2.54) (size 1.55 1.55) (drill 1) (layers *.Cu *.Mask) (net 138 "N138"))
  (pad B21 thru_hole circle (at 50.8 -2.54) (size 1.55 1.55) (drill 1) (layers *.Cu *.Mask) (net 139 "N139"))
  (pad B20 thru_hole circle (at 48.26 -2.54) (size 1.55 1.55) (drill 1) (layers *.Cu *.Mask) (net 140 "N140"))
  (pad B19 thru_hole circle (at 45.72 -2.54) (size 1.55 1.55) (drill 1) (layers *.Cu *.Mask) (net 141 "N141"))
  (pad B18 thru_hole circle (at 43.18 -2.54) (size 1.55 1.55) (drill 1) (layers *.Cu *.Mask) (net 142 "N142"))
  (pad B17 thru_hole circle (at 40.64 -2.54) (size 1.55 1.55) (drill 1) (layers *.Cu *.Mask) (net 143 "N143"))
  (pad B16 thru_hole circle (at 38.1 -2.54) (size 1.55 1.55) (drill 1) (layers *.Cu *.Mask) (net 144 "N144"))
  (pad B15 thru_hole circle (at 35.56 -2.54) (size 1.55 1.55) (drill 1) (layers *.Cu *.Mask) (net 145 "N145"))
  (pad B14 thru_hole circle (at 33.02 -2.54) (size 1.55 1.55) (drill 1) (layers *.Cu *.Mask) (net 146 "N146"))
  (pad B13 thru_hole circle (at 30.48 -2.54) (size 1.55 1.55) (drill 1) (layers *.Cu *.Mask) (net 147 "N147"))
  (pad B12 thru_hole circle (at 27.94 -2.54) (size 1.55 1.55) (drill 1) (layers *.Cu *.Mask) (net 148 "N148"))
  (pad B11 thru_hole circle (at 25.4 -2.54) (size 1.55 1.55) (drill 1) (layers *.Cu *.Mask) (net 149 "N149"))
  (pad B10 thru_hole circle (at 22.86 -2.54) (size 1.55 1.55) (drill 1) (layers *.Cu *.Mask) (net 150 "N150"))
  (pad B9 thru_hole circle (at 20.32 -2.54) (size 1.55 1.55) (drill 1) (layers *.Cu *.Mask) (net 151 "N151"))
  (pad B8 thru_hole circle (at 17.78 -2.54) (size 1.55 1.55) (drill 1) (layers *.Cu *.Mask) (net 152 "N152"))
  (pad B7 thru_hole circle (at 15.24 -2.54) (size 1.55 1.55) (drill 1) (layers *.Cu *.Mask) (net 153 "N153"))
  (pad B6 thru_hole circle (at 12.7 -2.54) (size 1.55 1.55) (drill 1) (layers *.Cu *.Mask) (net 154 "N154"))
  (pad B5 thru_hole circle (at 10.16 -2.54) (size 1.55 1.55) (drill 1) (layers *.Cu *.Mask) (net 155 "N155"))
  (pad B4 thru_hole circle (at 7.62 -2.54) (size 1.55 1.55) (drill 1) (layers *.Cu *.Mask) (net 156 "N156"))
  (pad B3 thru_hole circle (at 5.08 -2.54) (size 1.55 1.55) (drill 1) (layers *.Cu *.Mask) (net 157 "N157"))
  (pad B2 thru_hole circle (at 2.54 -2.54) (size 1.55 1.55) (drill 1) (layers *.Cu *.Mask) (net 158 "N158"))
  (pad B1 thru_hole circle (at 0 -2.54) (size 1.55 1.55) (drill 1) (layers *.Cu *.Mask) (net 64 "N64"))
  (pad A32 thru_hole circle (at 78.74 0) (size 1.55 1.55) (drill 1) (layers *.Cu *.Mask) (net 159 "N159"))
  (pad A31 thru_hole circle (at 76.2 0) (size 1.55 1.55) (drill 1) (layers *.Cu *.Mask) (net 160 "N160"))
  (pad A30 thru_hole circle (at 73.66 0) (size 1.55 1.55) (drill 1) (layers *.Cu *.Mask) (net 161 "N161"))
  (pad A29 thru_hole circle (at 71.12 0) (size 1.55 1.55) (drill 1) (layers *.Cu *.Mask) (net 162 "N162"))
  (pad A28 thru_hole circle (at 68.58 0) (size 1.55 1.55) (drill 1) (layers *.Cu *.Mask) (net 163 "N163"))
  (pad A27 thru_hole circle (at 66.04 0) (size 1.55 1.55) (drill 1) (layers *.Cu *.Mask) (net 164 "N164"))
  (pad A26 thru_hole circle (at 63.5 0) (size 1.55 1.55) (drill 1) (layers *.Cu *.Mask) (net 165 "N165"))
  (pad A25 thru_hole circle (at 60.96 0) (size 1.55 1.55) (drill 1) (layers *.Cu *.Mask) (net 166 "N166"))
  (pad A24 thru_hole circle (at 58.42 0) (size 1.55 1.55) (drill 1) (layers *.Cu *.Mask) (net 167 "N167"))
  (pad A23 thru_hole circle (at 55.88 0) (size 1.55 1.55) (drill 1) (layers *.Cu *.Mask) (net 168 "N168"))
  (pad A22 thru_hole circle (at 53.34 0) (size 1.55 1.55) (drill 1) (layers *.Cu *.Mask) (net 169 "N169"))
  (pad A21 thru_hole circle (at 50.8 0) (size 1.55 1.55) (drill 1) (layers *.Cu *.Mask) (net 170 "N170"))
  (pad A20 thru_hole circle (at 48.26 0) (size 1.55 1.55) (drill 1) (layers *.Cu *.Mask) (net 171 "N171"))
  (pad A19 thru_hole circle (at 45.72 0) (size 1.55 1.55) (drill 1) (layers *.Cu *.Mask) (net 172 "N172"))
  (pad A18 thru_hole circle (at 43.18 0) (size 1.55 1.55) (drill 1) (layers *.Cu *.Mask) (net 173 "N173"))
  (pad A17 thru_hole circle (at 40.64 0) (size 1.55 1.55) (drill 1) (layers *.Cu *.Mask) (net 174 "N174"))
  (pad A16 thru_hole circle (at 38.1 0) (size 1.55 1.55) (drill 1) (layers *.Cu *.Mask) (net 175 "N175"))
  (pad A15 thru_hole circle (at 35.56 0) (size 1.55 1.55) (drill 1) (layers *.Cu *.Mask) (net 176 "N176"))
  (pad A14 thru_hole circle (at 33.02 0) (size 1.55 1.55) (drill 1) (layers *.Cu *.Mask) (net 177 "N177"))
  (pad A13 thru_hole circle (at 30.48 0) (size 1.55 1.55) (drill 1) (layers *.Cu *.Mask) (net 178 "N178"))
  (pad A12 thru_hole circle (at 27.94 0) (size 1.55 1.55) (drill 1) (layers *.Cu *.Mask) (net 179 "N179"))
  (pad A11 thru_hole circle (at 25.4 0) (size 1.55 1.55) (drill 1) (layers *.Cu *.Mask) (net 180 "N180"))
  (pad A10 thru_hole circle (at 22.86 0) (size 1.55 1.55) (drill 1) (layers *.Cu *.Mask) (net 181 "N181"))
  (pad A9 thru_hole circle (at 20.32 0) (size 1.55 1.55) (drill 1) (layers *.Cu *.Mask) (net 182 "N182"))
  (pad A8 thru_hole circle (at 17.78 0) (size 1.55 1.55) (drill 1) (layers *.Cu *.Mask) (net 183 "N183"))
  (pad A7 thru_hole circle (at 15.24 0) (size 1.55 1.55) (drill 1) (layers *.Cu *.Mask) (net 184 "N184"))
  (pad A6 thru_hole circle (at 12.7 0) (size 1.55 1.55) (drill 1) (layers *.Cu *.Mask) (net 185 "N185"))
  (pad A5 thru_hole circle (at 10.16 0) (size 1.55 1.55) (drill 1) (layers *.Cu *.Mask) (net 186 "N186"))
  (pad A4 thru_hole circle (at 7.62 0) (size 1.55 1.55) (drill 1) (layers *.Cu *.Mask) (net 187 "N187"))
  (pad A3 thru_hole circle (at 5.08 0) (size 1.55 1.55) (drill 1) (layers *.Cu *.Mask) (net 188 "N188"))
  (pad A2 thru_hole circle (at 2.54 0) (size 1.55 1.55) (drill 1) (layers *.Cu *.Mask) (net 95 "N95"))
  (pad A1 thru_hole roundrect (at 0 0 270) (size 1.55 1.55) (drill 1) (layers *.Cu *.Mask) (roundrect_rratio 0.161) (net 96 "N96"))
  (pad "" np_thru_hole circle (at 83.82 2.54) (size 2.85 2.85) (drill 2.85) (layers *.Cu *.Mask))
  (pad "" np_thru_hole circle (at -5.08 2.54) (size 2.85 2.85) (drill 2.85) (layers *.Cu *.Mask)))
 (gr_line (start 99.8 66.3) (end 99.8 40.3) (layer Edge.Cuts) (width 0.05))
 (gr_line (start 199.8 66.3) (end 99.8 66.3) (layer Edge.Cuts) (width 0.05))
 (gr_line (start 199.8 40.3) (end 199.8 66.3) (layer Edge.Cuts) (width 0.05))
 (gr_line (start 99.8 40.3) (end 199.8 40.3) (layer Edge.Cuts) (width 0.05))
 (segment (start 110.43 55.92) (end 110.43 50.68) (width 0.25) (layer F.Cu) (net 32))
 (segment (start 111.869999 49.579999) (end 110.43 48.14) (width 0.25) (layer F.Cu) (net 64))
 (segment (start 111.869999 57.020001) (end 111.869999 49.579999) (width 0.25) (layer F.Cu) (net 64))
 (segment (start 110.43 58.46) (end 111.869999 57.020001) (width 0.25) (layer F.Cu) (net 64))
 (segment (start 109.329999 46.700001) (end 110.43 45.6) (width 0.25) (layer F.Cu) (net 96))
 (segment (start 109.329999 59.899999) (end 109.329999 46.700001) (width 0.25) (layer F.Cu) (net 96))
 (segment (start 110.43 61) (end 109.329999 59.899999) (width 0.25) (layer F.Cu) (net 96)))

